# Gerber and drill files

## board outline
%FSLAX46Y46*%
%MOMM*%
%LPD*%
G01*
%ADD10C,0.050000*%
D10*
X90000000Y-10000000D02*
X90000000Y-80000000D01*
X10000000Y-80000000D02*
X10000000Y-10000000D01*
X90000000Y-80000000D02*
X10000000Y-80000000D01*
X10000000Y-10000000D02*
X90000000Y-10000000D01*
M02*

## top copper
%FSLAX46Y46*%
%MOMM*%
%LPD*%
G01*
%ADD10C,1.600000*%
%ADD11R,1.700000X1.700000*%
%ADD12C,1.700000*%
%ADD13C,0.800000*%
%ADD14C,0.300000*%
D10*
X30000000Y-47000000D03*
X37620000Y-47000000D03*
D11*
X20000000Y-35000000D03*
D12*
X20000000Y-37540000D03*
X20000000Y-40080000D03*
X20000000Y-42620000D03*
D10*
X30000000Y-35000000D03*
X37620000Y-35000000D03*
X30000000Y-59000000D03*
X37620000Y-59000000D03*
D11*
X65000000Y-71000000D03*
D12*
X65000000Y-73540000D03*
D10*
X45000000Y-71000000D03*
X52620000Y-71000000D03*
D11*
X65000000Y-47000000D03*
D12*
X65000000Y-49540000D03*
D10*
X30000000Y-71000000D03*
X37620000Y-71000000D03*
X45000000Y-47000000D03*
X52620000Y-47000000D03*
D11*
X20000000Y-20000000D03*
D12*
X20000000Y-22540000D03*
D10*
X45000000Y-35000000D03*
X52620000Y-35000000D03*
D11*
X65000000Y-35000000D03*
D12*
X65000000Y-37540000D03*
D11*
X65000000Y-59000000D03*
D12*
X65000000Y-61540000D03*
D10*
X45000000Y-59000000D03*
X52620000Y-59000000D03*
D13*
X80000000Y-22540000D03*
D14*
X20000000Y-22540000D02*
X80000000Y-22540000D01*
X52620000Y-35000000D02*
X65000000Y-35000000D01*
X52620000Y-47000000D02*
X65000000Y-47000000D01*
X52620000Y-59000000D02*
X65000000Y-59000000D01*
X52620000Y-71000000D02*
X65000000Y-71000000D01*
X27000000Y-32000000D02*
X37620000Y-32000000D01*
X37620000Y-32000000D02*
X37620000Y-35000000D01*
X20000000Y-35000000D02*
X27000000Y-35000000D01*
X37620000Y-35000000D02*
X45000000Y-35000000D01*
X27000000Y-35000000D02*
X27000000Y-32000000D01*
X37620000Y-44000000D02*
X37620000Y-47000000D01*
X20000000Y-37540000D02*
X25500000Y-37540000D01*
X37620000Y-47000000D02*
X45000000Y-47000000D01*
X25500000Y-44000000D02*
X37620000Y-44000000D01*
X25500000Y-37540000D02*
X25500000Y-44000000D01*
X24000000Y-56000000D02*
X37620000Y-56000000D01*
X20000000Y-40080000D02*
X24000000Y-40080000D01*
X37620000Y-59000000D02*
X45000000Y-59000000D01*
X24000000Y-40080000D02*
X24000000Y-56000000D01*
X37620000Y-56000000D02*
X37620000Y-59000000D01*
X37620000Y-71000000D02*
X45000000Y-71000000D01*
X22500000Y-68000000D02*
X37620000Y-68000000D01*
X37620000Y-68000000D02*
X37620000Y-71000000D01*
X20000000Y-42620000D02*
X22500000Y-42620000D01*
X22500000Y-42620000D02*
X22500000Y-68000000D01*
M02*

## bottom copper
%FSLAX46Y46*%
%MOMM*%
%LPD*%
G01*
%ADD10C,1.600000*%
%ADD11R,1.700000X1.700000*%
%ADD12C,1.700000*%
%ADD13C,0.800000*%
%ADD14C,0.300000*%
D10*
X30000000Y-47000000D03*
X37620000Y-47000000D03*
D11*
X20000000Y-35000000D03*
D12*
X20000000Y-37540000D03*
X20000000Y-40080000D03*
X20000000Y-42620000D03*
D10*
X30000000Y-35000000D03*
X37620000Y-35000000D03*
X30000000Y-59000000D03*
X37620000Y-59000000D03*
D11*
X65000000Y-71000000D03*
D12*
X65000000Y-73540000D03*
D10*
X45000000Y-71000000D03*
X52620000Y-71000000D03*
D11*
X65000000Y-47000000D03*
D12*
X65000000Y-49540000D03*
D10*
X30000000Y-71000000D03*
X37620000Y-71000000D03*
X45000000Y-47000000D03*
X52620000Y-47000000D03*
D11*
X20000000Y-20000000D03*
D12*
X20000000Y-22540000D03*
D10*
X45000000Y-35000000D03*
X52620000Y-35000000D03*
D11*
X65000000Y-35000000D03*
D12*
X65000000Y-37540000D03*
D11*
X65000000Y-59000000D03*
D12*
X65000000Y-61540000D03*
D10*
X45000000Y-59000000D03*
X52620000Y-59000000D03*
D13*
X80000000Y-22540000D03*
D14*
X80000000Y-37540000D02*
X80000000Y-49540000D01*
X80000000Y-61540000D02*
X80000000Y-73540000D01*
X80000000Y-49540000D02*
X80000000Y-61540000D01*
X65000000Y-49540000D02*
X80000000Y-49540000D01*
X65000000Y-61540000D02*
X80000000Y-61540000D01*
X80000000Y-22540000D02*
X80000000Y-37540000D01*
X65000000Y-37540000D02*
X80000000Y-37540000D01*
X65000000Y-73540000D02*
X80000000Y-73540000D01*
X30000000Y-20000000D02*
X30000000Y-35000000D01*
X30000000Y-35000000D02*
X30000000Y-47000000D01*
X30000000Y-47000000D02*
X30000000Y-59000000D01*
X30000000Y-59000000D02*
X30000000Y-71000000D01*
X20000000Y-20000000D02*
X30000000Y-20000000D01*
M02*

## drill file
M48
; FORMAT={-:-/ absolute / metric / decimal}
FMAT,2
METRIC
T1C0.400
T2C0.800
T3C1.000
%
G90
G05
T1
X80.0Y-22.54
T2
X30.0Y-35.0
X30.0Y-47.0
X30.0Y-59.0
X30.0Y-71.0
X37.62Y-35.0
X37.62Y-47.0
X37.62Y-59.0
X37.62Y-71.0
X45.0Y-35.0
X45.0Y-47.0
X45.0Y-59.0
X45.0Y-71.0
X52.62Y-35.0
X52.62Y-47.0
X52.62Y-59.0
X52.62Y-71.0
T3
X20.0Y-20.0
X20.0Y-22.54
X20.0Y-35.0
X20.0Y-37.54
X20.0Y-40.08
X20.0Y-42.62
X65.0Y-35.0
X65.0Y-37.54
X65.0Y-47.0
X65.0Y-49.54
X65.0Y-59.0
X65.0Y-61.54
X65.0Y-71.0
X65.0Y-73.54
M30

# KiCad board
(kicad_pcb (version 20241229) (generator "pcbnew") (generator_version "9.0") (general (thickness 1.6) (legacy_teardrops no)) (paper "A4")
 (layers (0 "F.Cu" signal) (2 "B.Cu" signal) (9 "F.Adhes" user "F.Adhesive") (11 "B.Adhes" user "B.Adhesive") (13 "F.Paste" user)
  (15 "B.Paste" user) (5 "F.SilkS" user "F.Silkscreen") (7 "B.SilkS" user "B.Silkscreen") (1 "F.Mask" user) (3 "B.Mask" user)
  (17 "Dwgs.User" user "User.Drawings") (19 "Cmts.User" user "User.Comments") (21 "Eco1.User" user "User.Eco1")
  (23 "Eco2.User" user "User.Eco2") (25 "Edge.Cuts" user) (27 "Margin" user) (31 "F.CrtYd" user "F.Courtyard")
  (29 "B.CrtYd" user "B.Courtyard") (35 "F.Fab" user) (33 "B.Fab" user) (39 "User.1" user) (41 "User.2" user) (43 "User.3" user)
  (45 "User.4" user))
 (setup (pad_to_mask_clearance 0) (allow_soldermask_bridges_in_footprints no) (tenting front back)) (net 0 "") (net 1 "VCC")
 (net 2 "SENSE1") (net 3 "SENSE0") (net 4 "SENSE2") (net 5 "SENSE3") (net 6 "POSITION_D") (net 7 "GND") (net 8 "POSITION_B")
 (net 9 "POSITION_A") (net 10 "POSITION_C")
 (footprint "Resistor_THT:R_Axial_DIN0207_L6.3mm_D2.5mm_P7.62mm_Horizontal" (layer "F.Cu") (at 30 47)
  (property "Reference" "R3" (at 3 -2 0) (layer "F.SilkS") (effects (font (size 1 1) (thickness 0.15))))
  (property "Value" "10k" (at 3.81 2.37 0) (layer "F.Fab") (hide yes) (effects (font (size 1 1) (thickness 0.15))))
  (pad "1" thru_hole circle (at 0 0) (size 1.6 1.6) (drill 0.8) (layers "*.Cu" "*.Mask") (remove_unused_layers no) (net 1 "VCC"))
  (pad "2" thru_hole circle (at 7.62 0) (size 1.6 1.6) (drill 0.8) (layers "*.Cu" "*.Mask") (remove_unused_layers no) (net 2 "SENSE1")))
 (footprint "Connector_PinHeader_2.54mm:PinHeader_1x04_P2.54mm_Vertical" (layer "F.Cu") (at 20 35)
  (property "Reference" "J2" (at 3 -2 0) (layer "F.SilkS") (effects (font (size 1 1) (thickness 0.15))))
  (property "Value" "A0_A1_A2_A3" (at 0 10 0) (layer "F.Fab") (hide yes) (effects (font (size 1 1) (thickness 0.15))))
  (pad "1" thru_hole rect (at 0 0) (size 1.7 1.7) (drill 1) (layers "*.Cu" "*.Mask") (remove_unused_layers no) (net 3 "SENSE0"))
  (pad "2" thru_hole circle (at 0 2.54) (size 1.7 1.7) (drill 1) (layers "*.Cu" "*.Mask") (remove_unused_layers no) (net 2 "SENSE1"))
  (pad "3" thru_hole circle (at 0 5.08) (size 1.7 1.7) (drill 1) (layers "*.Cu" "*.Mask") (remove_unused_layers no) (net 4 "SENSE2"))
  (pad "4" thru_hole circle (at 0 7.62) (size 1.7 1.7) (drill 1) (layers "*.Cu" "*.Mask") (remove_unused_layers no) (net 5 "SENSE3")))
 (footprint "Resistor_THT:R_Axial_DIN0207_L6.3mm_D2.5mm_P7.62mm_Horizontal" (layer "F.Cu") (at 30 35)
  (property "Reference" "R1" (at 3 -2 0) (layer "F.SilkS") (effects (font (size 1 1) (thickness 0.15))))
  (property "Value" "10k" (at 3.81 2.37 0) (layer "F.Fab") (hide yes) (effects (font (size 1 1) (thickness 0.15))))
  (pad "1" thru_hole circle (at 0 0) (size 1.6 1.6) (drill 0.8) (layers "*.Cu" "*.Mask") (remove_unused_layers no) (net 1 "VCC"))
  (pad "2" thru_hole circle (at 7.62 0) (size 1.6 1.6) (drill 0.8) (layers "*.Cu" "*.Mask") (remove_unused_layers no) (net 3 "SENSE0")))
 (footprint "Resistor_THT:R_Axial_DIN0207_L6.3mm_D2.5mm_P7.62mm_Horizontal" (layer "F.Cu") (at 30 59)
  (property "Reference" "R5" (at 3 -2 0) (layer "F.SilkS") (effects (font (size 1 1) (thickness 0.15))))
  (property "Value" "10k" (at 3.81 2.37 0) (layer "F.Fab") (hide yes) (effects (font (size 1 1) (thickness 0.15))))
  (pad "1" thru_hole circle (at 0 0) (size 1.6 1.6) (drill 0.8) (layers "*.Cu" "*.Mask") (remove_unused_layers no) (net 1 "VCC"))
  (pad "2" thru_hole circle (at 7.62 0) (size 1.6 1.6) (drill 0.8) (layers "*.Cu" "*.Mask") (remove_unused_layers no) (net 4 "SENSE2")))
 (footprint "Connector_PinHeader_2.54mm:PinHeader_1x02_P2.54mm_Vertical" (layer "F.Cu") (at 65 71)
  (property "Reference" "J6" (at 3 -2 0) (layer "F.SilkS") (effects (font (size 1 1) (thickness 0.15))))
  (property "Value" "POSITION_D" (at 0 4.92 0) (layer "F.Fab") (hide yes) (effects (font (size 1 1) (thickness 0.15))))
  (pad "1" thru_hole rect (at 0 0) (size 1.7 1.7) (drill 1) (layers "*.Cu" "*.Mask") (remove_unused_layers no) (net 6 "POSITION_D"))
  (pad "2" thru_hole circle (at 0 2.54) (size 1.7 1.7) (drill 1) (layers "*.Cu" "*.Mask") (remove_unused_layers no) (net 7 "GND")))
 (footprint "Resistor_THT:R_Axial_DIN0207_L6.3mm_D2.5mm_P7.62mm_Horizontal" (layer "F.Cu") (at 45 71)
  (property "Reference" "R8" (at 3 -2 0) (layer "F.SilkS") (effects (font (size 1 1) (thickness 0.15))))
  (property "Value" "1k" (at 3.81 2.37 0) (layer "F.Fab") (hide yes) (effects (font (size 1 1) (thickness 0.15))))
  (pad "1" thru_hole circle (at 0 0) (size 1.6 1.6) (drill 0.8) (layers "*.Cu" "*.Mask") (remove_unused_layers no) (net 5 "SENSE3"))
  (pad "2" thru_hole circle (at 7.62 0) (size 1.6 1.6) (drill 0.8) (layers "*.Cu" "*.Mask") (remove_unused_layers no) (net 6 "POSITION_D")))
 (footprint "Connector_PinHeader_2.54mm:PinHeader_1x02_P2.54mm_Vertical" (layer "F.Cu") (at 65 47)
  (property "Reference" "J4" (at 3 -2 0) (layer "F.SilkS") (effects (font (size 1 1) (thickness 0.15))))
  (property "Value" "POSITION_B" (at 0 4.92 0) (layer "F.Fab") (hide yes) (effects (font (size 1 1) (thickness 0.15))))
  (pad "1" thru_hole rect (at 0 0) (size 1.7 1.7) (drill 1) (layers "*.Cu" "*.Mask") (remove_unused_layers no) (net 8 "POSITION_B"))
  (pad "2" thru_hole circle (at 0 2.54) (size 1.7 1.7) (drill 1) (layers "*.Cu" "*.Mask") (remove_unused_layers no) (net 7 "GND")))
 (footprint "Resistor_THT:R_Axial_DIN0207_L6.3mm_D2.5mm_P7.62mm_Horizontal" (layer "F.Cu") (at 30 71)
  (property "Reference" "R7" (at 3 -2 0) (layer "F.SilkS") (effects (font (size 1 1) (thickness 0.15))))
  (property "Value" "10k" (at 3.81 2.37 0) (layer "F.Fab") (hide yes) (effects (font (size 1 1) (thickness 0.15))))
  (pad "1" thru_hole circle (at 0 0) (size 1.6 1.6) (drill 0.8) (layers "*.Cu" "*.Mask") (remove_unused_layers no) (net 1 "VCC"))
  (pad "2" thru_hole circle (at 7.62 0) (size 1.6 1.6) (drill 0.8) (layers "*.Cu" "*.Mask") (remove_unused_layers no) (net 5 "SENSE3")))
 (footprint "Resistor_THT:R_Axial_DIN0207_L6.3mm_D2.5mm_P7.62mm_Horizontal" (layer "F.Cu") (at 45 47)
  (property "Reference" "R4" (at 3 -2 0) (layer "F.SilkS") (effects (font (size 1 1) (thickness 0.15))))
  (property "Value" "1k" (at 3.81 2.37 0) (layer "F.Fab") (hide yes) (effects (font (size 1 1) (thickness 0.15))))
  (pad "1" thru_hole circle (at 0 0) (size 1.6 1.6) (drill 0.8) (layers "*.Cu" "*.Mask") (remove_unused_layers no) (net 2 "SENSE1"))
  (pad "2" thru_hole circle (at 7.62 0) (size 1.6 1.6) (drill 0.8) (layers "*.Cu" "*.Mask") (remove_unused_layers no) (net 8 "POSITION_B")))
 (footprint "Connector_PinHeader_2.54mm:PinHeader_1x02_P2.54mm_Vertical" (layer "F.Cu") (at 20 20)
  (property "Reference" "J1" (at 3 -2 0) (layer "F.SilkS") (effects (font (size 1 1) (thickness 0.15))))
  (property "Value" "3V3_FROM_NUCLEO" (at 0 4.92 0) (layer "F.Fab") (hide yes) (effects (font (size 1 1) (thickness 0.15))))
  (pad "1" thru_hole rect (at 0 0) (size 1.7 1.7) (drill 1) (layers "*.Cu" "*.Mask") (remove_unused_layers no) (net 1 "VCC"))
  (pad "2" thru_hole circle (at 0 2.54) (size 1.7 1.7) (drill 1) (layers "*.Cu" "*.Mask") (remove_unused_layers no) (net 7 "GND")))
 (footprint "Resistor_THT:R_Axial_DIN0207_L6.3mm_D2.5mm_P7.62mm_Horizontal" (layer "F.Cu") (at 45 35)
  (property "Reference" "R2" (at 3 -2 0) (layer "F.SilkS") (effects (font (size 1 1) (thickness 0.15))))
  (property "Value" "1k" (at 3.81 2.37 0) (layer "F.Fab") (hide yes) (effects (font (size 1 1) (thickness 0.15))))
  (pad "1" thru_hole circle (at 0 0) (size 1.6 1.6) (drill 0.8) (layers "*.Cu" "*.Mask") (remove_unused_layers no) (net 3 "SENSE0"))
  (pad "2" thru_hole circle (at 7.62 0) (size 1.6 1.6) (drill 0.8) (layers "*.Cu" "*.Mask") (remove_unused_layers no) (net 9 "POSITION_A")))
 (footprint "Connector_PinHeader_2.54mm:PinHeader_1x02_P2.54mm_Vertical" (layer "F.Cu") (at 65 35)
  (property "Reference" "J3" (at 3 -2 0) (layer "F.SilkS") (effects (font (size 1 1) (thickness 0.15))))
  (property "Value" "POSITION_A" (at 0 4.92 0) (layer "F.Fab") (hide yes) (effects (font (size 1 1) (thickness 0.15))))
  (pad "1" thru_hole rect (at 0 0) (size 1.7 1.7) (drill 1) (layers "*.Cu" "*.Mask") (remove_unused_layers no) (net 9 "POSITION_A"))
  (pad "2" thru_hole circle (at 0 2.54) (size 1.7 1.7) (drill 1) (layers "*.Cu" "*.Mask") (remove_unused_layers no) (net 7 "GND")))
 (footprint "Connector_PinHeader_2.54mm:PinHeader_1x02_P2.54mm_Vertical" (layer "F.Cu") (at 65 59)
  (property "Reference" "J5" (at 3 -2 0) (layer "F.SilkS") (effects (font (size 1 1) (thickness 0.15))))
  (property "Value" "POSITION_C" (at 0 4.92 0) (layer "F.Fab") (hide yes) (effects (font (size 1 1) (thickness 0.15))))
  (pad "1" thru_hole rect (at 0 0) (size 1.7 1.7) (drill 1) (layers "*.Cu" "*.Mask") (remove_unused_layers no) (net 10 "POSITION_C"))
  (pad "2" thru_hole circle (at 0 2.54) (size 1.7 1.7) (drill 1) (layers "*.Cu" "*.Mask") (remove_unused_layers no) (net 7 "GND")))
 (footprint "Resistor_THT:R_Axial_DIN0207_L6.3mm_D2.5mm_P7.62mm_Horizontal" (layer "F.Cu") (at 45 59)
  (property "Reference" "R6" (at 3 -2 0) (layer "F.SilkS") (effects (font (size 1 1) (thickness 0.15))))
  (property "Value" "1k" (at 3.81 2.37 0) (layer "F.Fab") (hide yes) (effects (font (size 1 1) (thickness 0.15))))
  (pad "1" thru_hole circle (at 0 0) (size 1.6 1.6) (drill 0.8) (layers "*.Cu" "*.Mask") (remove_unused_layers no) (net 4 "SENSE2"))
  (pad "2" thru_hole circle (at 7.62 0) (size 1.6 1.6) (drill 0.8) (layers "*.Cu" "*.Mask") (remove_unused_layers no) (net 10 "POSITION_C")))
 (gr_line (start 90 10) (end 90 80) (stroke (width 0.05) (type default)) (layer "Edge.Cuts"))
 (gr_line (start 10 80) (end 10 10) (stroke (width 0.05) (type default)) (layer "Edge.Cuts"))
 (gr_line (start 90 80) (end 10 80) (stroke (width 0.05) (type default)) (layer "Edge.Cuts"))
 (gr_line (start 10 10) (end 90 10) (stroke (width 0.05) (type default)) (layer "Edge.Cuts"))
 (segment (start 20 22.54) (end 80 22.54) (width 0.3) (layer "F.Cu") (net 7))
 (via (at 80 22.54) (size 0.8) (drill 0.4) (layers "F.Cu" "B.Cu") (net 7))
 (segment (start 80 37.54) (end 80 49.54) (width 0.3) (layer "B.Cu") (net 7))
 (segment (start 80 61.54) (end 80 73.54) (width 0.3) (layer "B.Cu") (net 7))
 (segment (start 80 49.54) (end 80 61.54) (width 0.3) (layer "B.Cu") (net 7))
 (segment (start 65 49.54) (end 80 49.54) (width 0.3) (layer "B.Cu") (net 7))
 (segment (start 65 61.54) (end 80 61.54) (width 0.3) (layer "B.Cu") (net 7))
 (segment (start 80 22.54) (end 80 37.54) (width 0.3) (layer "B.Cu") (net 7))
 (segment (start 65 37.54) (end 80 37.54) (width 0.3) (layer "B.Cu") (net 7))
 (segment (start 65 73.54) (end 80 73.54) (width 0.3) (layer "B.Cu") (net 7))
 (segment (start 52.62 35) (end 65 35) (width 0.3) (layer "F.Cu") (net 9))
 (segment (start 52.62 47) (end 65 47) (width 0.3) (layer "F.Cu") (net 8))
 (segment (start 52.62 59) (end 65 59) (width 0.3) (layer "F.Cu") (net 10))
 (segment (start 52.62 71) (end 65 71) (width 0.3) (layer "F.Cu") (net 6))
 (segment (start 27 32) (end 37.62 32) (width 0.3) (layer "F.Cu") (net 3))
 (segment (start 37.62 32) (end 37.62 35) (width 0.3) (layer "F.Cu") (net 3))
 (segment (start 20 35) (end 27 35) (width 0.3) (layer "F.Cu") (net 3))
 (segment (start 37.62 35) (end 45 35) (width 0.3) (layer "F.Cu") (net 3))
 (segment (start 27 35) (end 27 32) (width 0.3) (layer "F.Cu") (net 3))
 (segment (start 37.62 44) (end 37.62 47) (width 0.3) (layer "F.Cu") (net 2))
 (segment (start 20 37.54) (end 25.5 37.54) (width 0.3) (layer "F.Cu") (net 2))
 (segment (start 37.62 47) (end 45 47) (width 0.3) (layer "F.Cu") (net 2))
 (segment (start 25.5 44) (end 37.62 44) (width 0.3) (layer "F.Cu") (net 2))
 (segment (start 25.5 37.54) (end 25.5 44) (width 0.3) (layer "F.Cu") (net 2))
 (segment (start 24 56) (end 37.62 56) (width 0.3) (layer "F.Cu") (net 4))
 (segment (start 20 40.08) (end 24 40.08) (width 0.3) (layer "F.Cu") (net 4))
 (segment (start 37.62 59) (end 45 59) (width 0.3) (layer "F.Cu") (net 4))
 (segment (start 24 40.08) (end 24 56) (width 0.3) (layer "F.Cu") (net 4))
 (segment (start 37.62 56) (end 37.62 59) (width 0.3) (layer "F.Cu") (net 4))
 (segment (start 37.62 71) (end 45 71) (width 0.3) (layer "F.Cu") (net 5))
 (segment (start 22.5 68) (end 37.62 68) (width 0.3) (layer "F.Cu") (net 5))
 (segment (start 37.62 68) (end 37.62 71) (width 0.3) (layer "F.Cu") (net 5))
 (segment (start 20 42.62) (end 22.5 42.62) (width 0.3) (layer "F.Cu") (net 5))
 (segment (start 22.5 42.62) (end 22.5 68) (width 0.3) (layer "F.Cu") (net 5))
 (segment (start 30 20) (end 30 35) (width 0.3) (layer "B.Cu") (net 1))
 (segment (start 30 35) (end 30 47) (width 0.3) (layer "B.Cu") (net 1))
 (segment (start 30 47) (end 30 59) (width 0.3) (layer "B.Cu") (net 1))
 (segment (start 30 59) (end 30 71) (width 0.3) (layer "B.Cu") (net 1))
 (segment (start 20 20) (end 30 20) (width 0.3) (layer "B.Cu") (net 1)))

